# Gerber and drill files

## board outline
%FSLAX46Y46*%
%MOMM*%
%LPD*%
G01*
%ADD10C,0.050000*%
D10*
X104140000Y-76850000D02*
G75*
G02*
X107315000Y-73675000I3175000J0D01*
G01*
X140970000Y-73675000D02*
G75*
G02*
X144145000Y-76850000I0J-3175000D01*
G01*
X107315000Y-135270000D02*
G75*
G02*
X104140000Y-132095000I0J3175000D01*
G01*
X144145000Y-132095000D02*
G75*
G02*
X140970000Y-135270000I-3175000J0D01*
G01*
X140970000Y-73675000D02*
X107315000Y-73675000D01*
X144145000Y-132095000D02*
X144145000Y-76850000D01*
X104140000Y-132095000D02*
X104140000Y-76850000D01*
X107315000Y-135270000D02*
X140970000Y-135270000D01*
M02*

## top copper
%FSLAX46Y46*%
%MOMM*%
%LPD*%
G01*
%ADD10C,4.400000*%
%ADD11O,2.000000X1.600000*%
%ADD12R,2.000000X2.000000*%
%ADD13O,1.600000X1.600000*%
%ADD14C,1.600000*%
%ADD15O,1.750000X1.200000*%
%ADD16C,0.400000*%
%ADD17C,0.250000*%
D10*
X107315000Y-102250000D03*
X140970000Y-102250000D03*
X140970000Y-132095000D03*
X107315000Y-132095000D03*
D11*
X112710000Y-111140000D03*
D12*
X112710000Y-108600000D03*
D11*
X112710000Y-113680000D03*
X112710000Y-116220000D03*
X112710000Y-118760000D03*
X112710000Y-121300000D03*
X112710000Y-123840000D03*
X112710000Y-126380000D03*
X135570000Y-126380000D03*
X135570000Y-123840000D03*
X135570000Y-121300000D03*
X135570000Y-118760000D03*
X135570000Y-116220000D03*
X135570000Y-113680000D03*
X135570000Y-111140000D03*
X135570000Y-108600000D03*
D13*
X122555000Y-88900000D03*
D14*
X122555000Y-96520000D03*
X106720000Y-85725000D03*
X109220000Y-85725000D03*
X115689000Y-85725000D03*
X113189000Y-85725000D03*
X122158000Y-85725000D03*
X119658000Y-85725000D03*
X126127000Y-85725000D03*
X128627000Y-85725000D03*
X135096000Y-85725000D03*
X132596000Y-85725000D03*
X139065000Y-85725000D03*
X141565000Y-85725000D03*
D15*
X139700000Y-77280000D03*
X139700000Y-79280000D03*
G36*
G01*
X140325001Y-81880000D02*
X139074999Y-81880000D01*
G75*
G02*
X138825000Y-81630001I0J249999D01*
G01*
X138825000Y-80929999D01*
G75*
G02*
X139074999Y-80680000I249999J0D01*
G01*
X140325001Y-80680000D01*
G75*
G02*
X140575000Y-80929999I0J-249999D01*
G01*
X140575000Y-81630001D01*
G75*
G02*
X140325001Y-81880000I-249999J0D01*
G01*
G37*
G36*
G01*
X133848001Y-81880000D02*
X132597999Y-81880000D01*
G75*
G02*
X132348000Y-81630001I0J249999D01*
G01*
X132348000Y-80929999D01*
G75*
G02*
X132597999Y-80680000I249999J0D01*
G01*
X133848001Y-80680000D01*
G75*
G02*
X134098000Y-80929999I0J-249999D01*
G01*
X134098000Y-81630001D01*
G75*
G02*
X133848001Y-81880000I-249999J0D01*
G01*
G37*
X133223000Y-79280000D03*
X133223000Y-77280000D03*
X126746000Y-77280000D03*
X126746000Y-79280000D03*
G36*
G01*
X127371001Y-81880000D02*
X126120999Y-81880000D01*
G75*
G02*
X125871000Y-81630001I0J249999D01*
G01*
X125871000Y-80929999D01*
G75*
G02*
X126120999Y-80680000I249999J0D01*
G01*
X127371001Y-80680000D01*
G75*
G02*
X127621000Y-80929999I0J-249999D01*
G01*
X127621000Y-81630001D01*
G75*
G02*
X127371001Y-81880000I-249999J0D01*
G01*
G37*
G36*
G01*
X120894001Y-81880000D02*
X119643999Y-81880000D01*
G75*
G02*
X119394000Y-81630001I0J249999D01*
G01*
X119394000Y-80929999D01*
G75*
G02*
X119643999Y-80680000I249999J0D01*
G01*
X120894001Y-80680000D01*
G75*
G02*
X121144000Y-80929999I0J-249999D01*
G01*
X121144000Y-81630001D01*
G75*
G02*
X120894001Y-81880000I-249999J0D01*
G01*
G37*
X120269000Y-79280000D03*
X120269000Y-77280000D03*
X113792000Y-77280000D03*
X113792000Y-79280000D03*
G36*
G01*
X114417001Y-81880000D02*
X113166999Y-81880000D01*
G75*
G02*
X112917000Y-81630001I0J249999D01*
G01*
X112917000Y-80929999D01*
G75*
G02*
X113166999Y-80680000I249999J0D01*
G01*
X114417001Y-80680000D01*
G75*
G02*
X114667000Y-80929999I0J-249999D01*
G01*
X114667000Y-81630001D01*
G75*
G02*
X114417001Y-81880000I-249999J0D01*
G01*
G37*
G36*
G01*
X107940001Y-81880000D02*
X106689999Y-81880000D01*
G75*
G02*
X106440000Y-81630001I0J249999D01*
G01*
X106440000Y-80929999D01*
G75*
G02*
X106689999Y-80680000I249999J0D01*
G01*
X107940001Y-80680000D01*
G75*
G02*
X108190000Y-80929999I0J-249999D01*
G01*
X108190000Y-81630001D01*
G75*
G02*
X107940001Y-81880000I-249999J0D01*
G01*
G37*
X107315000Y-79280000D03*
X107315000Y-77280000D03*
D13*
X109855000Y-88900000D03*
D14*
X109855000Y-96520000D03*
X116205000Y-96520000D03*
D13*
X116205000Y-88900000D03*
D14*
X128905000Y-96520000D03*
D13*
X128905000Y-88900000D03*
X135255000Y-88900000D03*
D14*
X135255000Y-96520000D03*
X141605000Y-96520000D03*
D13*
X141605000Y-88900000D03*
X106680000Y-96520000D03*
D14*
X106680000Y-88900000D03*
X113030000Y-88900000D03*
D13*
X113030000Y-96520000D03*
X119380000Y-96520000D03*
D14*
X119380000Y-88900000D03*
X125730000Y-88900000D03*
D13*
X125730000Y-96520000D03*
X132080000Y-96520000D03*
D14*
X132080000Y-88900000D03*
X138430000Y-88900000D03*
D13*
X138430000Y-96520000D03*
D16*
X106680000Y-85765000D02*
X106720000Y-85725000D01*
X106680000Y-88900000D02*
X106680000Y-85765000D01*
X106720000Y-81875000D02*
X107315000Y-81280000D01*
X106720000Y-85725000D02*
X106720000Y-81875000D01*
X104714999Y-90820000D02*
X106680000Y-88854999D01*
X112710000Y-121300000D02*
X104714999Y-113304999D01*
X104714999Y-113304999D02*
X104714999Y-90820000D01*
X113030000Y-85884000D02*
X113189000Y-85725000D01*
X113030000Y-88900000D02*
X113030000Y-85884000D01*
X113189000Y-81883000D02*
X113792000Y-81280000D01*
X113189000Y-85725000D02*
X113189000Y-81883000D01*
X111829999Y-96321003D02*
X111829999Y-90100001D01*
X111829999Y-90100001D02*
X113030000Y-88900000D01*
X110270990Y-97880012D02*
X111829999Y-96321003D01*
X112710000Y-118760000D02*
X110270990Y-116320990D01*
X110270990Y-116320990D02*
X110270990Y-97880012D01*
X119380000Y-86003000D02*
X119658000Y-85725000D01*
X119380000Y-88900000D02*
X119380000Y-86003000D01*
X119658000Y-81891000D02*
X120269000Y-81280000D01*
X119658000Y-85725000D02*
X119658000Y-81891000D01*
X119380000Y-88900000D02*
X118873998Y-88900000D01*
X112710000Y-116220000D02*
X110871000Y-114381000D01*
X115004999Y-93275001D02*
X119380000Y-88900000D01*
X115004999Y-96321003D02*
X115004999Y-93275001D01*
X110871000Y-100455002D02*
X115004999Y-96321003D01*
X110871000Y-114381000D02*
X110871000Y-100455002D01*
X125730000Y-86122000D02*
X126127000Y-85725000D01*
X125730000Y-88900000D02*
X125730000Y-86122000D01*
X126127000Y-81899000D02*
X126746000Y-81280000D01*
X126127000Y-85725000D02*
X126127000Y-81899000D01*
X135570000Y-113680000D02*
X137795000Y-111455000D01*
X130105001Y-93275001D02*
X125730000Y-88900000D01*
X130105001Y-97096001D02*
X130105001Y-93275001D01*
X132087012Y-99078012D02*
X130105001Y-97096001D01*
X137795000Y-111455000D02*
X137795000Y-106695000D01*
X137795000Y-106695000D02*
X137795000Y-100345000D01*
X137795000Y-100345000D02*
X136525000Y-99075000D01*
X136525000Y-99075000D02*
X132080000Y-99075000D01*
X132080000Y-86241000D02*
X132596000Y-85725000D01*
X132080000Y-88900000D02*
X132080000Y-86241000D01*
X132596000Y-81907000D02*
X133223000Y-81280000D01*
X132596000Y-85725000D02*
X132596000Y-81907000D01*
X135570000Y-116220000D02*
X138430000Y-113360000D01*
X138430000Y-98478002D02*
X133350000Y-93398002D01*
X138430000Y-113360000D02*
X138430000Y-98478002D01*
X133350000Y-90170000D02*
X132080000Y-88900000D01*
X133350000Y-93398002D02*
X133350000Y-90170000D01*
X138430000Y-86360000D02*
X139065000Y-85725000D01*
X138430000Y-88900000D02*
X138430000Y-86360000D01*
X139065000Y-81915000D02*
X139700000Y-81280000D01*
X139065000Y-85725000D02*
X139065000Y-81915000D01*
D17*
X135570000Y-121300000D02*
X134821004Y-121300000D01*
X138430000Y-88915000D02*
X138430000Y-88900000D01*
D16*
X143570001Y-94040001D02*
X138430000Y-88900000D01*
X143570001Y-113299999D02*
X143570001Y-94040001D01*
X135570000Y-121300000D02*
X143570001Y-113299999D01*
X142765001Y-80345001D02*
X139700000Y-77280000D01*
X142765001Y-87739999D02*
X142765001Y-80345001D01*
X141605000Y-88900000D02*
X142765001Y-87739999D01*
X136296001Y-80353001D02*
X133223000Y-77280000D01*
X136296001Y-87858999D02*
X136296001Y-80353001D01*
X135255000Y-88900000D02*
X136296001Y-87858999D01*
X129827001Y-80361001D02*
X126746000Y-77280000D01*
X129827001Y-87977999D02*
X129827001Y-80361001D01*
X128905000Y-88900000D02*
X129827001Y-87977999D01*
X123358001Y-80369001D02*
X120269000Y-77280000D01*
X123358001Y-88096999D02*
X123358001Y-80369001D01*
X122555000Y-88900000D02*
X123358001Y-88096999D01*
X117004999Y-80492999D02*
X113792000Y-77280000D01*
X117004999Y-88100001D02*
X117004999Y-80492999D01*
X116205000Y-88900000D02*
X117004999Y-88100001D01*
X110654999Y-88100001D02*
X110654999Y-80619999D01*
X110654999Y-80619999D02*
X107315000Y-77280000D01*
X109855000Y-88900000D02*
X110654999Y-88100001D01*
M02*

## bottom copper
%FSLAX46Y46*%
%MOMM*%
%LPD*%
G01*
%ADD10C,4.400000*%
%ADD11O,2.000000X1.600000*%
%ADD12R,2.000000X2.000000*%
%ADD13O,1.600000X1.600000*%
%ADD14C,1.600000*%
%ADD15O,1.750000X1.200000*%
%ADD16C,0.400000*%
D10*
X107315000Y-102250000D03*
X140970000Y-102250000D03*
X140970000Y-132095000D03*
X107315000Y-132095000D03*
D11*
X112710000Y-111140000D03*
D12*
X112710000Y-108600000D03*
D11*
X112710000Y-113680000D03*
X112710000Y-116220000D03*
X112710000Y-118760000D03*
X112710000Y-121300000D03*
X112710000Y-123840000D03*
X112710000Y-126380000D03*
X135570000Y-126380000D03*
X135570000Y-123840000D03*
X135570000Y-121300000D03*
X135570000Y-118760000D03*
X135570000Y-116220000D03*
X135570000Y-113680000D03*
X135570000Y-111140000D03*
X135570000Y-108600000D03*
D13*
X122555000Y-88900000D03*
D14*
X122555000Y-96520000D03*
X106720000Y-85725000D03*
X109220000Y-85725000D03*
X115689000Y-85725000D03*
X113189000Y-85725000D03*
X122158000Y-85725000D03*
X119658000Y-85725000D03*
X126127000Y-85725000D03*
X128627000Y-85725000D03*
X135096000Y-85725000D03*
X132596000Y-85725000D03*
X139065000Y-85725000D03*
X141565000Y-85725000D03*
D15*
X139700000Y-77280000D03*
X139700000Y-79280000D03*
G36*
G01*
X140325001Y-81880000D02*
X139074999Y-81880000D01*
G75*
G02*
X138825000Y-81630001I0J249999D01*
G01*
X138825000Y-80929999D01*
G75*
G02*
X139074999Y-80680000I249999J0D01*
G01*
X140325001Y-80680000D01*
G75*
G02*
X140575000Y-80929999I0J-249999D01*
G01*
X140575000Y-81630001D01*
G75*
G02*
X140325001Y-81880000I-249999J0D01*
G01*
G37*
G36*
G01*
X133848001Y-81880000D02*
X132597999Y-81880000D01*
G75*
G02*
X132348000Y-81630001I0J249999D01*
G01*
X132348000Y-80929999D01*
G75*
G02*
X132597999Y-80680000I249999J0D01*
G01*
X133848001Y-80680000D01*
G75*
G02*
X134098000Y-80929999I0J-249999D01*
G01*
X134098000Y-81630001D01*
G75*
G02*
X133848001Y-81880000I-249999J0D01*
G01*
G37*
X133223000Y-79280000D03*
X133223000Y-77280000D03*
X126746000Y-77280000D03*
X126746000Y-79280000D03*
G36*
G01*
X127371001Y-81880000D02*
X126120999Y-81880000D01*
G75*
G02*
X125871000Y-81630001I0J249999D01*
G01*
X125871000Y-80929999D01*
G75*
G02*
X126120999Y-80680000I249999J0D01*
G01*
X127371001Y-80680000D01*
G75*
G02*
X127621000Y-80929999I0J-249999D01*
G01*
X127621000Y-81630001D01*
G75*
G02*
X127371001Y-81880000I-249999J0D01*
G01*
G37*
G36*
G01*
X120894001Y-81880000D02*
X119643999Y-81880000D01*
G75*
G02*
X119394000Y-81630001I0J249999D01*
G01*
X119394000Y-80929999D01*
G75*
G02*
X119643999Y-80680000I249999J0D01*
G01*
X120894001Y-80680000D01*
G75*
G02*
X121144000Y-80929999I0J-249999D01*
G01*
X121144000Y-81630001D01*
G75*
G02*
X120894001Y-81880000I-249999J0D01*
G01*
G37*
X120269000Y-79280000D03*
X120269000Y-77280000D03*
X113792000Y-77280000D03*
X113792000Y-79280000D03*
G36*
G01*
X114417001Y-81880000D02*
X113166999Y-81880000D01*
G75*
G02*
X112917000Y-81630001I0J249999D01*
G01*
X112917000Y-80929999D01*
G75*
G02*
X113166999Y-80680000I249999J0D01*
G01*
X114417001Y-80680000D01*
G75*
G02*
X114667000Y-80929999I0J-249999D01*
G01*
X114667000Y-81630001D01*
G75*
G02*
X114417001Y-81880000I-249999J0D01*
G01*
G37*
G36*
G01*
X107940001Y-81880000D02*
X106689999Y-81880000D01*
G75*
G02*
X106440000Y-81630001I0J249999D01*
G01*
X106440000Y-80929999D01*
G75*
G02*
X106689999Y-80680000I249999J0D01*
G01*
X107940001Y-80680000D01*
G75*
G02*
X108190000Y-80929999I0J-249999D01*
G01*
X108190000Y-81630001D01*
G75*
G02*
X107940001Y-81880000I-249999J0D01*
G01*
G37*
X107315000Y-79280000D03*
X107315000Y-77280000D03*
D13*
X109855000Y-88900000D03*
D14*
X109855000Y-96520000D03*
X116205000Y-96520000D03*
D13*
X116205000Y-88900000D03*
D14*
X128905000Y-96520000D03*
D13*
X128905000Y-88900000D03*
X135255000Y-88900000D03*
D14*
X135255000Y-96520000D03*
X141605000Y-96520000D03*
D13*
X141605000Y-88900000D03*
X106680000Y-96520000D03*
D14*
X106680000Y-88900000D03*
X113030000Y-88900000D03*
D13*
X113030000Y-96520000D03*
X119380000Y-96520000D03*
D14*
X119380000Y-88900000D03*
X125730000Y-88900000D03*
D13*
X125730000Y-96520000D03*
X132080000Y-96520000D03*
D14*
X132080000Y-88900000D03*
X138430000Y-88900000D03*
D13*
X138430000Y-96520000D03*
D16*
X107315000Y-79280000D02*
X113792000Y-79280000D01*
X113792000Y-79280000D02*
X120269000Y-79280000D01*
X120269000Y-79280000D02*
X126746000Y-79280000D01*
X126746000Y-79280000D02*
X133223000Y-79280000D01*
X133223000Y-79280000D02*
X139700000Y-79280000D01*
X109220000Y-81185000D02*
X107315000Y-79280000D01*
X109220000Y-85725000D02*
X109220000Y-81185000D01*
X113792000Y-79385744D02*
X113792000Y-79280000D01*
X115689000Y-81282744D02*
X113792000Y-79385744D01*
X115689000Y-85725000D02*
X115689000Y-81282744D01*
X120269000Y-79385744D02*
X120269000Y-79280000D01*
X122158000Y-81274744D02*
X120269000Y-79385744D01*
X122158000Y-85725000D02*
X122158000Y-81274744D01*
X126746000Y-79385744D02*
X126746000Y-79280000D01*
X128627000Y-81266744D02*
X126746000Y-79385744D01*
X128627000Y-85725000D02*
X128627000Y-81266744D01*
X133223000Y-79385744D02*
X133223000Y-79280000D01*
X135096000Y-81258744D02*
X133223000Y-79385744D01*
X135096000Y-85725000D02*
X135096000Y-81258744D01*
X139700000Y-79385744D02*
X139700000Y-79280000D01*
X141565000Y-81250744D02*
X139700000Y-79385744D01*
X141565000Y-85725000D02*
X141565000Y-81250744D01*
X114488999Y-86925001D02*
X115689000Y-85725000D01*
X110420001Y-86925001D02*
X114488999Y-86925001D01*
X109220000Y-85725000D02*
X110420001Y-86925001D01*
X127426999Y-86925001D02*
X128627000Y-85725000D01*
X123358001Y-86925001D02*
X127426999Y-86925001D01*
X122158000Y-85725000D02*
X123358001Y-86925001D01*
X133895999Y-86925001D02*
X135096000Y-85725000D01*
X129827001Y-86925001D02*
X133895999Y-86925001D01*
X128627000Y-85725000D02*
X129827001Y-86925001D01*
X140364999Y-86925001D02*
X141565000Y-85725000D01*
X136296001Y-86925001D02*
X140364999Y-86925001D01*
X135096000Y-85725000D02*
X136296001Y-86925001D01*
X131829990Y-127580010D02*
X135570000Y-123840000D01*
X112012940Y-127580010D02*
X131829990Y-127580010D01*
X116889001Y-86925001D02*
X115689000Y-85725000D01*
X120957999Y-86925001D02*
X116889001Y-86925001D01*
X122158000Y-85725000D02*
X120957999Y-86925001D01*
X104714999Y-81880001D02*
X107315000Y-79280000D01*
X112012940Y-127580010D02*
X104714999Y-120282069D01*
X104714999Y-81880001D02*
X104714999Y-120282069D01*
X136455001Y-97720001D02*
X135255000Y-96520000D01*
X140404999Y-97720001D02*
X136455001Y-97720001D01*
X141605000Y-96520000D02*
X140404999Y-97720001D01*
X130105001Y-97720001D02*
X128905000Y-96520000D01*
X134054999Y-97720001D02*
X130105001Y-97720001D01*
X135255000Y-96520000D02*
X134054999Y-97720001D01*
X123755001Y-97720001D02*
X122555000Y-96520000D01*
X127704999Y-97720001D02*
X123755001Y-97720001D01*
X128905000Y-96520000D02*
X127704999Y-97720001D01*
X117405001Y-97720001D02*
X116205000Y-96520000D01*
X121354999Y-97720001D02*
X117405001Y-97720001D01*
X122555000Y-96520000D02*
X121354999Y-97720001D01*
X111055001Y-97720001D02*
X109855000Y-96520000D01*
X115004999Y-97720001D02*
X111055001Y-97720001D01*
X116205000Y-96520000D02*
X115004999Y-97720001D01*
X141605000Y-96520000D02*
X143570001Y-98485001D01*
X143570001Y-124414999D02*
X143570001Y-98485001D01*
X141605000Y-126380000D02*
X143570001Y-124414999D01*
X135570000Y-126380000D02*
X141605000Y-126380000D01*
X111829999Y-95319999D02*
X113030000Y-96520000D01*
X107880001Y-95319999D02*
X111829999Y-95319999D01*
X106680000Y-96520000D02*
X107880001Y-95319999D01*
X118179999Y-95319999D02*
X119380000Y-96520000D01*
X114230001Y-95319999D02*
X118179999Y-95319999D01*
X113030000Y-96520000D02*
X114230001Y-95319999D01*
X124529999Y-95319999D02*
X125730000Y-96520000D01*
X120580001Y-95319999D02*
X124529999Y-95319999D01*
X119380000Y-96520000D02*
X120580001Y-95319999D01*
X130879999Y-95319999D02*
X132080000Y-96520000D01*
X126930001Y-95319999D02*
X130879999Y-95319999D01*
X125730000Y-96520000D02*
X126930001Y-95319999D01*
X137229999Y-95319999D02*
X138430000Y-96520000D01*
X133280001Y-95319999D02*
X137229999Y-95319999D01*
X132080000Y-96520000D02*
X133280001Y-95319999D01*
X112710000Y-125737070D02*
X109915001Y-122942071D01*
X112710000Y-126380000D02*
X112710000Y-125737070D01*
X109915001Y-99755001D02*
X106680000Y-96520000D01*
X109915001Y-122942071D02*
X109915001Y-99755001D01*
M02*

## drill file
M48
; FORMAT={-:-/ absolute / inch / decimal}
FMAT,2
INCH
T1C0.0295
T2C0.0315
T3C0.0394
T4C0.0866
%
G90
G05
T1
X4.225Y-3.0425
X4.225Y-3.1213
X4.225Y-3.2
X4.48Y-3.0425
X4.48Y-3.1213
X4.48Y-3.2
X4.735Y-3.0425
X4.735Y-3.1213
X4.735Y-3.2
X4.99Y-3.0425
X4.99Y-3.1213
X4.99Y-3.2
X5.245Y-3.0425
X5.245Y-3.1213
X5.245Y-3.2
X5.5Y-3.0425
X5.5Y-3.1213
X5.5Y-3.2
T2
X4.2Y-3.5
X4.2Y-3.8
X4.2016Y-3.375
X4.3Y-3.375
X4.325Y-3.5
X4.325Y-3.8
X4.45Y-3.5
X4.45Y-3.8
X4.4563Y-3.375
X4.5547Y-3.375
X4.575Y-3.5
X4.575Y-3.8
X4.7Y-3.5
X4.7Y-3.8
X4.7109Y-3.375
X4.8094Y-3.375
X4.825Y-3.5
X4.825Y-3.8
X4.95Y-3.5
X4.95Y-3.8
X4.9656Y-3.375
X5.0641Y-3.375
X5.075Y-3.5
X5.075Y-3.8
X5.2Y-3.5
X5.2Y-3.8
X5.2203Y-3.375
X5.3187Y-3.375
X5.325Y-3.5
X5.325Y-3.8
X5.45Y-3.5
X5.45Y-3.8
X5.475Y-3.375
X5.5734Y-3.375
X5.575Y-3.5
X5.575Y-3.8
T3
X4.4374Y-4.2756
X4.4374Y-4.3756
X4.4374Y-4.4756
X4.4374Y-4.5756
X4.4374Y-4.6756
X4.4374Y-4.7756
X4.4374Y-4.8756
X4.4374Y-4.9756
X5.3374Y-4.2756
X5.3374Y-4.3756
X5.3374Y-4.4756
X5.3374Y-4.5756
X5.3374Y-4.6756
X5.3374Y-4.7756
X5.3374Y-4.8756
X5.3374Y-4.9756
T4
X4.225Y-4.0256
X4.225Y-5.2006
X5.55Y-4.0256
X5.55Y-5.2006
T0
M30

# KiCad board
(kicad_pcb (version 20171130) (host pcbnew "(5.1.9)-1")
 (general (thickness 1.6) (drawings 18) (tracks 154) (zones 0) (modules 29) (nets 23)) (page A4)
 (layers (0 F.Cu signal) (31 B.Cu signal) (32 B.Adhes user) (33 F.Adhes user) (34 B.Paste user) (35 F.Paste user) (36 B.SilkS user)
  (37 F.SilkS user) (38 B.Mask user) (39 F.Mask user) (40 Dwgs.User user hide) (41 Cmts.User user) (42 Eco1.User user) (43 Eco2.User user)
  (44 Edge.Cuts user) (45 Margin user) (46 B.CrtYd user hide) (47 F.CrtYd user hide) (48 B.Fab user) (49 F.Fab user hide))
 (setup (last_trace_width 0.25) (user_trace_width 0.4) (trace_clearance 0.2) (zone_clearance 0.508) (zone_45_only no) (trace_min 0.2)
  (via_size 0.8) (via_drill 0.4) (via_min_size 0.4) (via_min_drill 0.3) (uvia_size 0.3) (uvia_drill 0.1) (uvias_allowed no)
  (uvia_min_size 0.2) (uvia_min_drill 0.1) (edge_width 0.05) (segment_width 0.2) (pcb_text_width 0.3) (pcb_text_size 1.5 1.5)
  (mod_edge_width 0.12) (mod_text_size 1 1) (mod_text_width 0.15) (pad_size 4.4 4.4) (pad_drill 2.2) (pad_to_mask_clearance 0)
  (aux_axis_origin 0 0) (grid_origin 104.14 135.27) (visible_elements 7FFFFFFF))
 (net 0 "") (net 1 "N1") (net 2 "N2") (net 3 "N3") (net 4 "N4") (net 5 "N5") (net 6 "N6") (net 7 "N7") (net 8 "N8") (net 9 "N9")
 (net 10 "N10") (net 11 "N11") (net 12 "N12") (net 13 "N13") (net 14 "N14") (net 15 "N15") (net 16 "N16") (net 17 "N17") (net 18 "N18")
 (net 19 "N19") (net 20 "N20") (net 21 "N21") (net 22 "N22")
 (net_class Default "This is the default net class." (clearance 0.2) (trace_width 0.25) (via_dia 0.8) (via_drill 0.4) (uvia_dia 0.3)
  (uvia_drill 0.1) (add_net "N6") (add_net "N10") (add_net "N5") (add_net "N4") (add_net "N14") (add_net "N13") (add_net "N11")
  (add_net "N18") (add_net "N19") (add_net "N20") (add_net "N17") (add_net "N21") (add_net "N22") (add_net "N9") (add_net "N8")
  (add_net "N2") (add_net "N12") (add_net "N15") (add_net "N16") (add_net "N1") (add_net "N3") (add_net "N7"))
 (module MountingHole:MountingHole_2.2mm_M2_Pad (layer F.Cu) (at 107.315 102.25)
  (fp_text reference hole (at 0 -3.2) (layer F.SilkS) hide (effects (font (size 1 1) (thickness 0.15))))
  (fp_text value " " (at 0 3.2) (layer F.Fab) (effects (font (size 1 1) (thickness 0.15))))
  (pad 4 thru_hole circle (at 0 0) (size 4.4 4.4) (drill 2.2) (layers *.Cu *.Mask)))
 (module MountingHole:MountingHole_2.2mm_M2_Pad (layer F.Cu) (at 140.97 102.25)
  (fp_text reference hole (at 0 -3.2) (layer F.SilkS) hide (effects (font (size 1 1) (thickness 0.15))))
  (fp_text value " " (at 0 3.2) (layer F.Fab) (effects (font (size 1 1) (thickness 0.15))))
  (pad 3 thru_hole circle (at 0 0) (size 4.4 4.4) (drill 2.2) (layers *.Cu *.Mask)))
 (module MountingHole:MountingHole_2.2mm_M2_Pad (layer F.Cu) (at 140.97 132.095)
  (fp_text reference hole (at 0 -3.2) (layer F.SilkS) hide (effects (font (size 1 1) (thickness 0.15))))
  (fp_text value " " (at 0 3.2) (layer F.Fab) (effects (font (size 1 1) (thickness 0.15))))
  (pad 2 thru_hole circle (at 0 0) (size 4.4 4.4) (drill 2.2) (layers *.Cu *.Mask)))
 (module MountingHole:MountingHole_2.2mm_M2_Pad (layer F.Cu) (at 107.315 132.095)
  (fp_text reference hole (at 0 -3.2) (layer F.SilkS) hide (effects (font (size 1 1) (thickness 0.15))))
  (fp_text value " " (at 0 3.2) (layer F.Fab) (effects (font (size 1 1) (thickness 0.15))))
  (pad 1 thru_hole circle (at 0 0) (size 4.4 4.4) (drill 2.2) (layers *.Cu *.Mask)))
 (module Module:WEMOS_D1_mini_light (layer F.Cu) (at 112.71 108.6)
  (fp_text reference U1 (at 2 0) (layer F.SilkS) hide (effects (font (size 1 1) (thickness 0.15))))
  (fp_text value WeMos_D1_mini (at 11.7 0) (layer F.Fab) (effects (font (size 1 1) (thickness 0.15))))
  (pad 2 thru_hole oval (at 0 2.54) (size 2 1.6) (drill 1) (layers *.Cu *.Mask) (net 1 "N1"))
  (pad 1 thru_hole rect (at 0 0) (size 2 2) (drill 1) (layers *.Cu *.Mask) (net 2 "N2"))
  (pad 3 thru_hole oval (at 0 5.08) (size 2 1.6) (drill 1) (layers *.Cu *.Mask) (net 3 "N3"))
  (pad 4 thru_hole oval (at 0 7.62) (size 2 1.6) (drill 1) (layers *.Cu *.Mask) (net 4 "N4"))
  (pad 5 thru_hole oval (at 0 10.16) (size 2 1.6) (drill 1) (layers *.Cu *.Mask) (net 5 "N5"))
  (pad 6 thru_hole oval (at 0 12.7) (size 2 1.6) (drill 1) (layers *.Cu *.Mask) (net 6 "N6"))
  (pad 7 thru_hole oval (at 0 15.24) (size 2 1.6) (drill 1) (layers *.Cu *.Mask) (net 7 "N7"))
  (pad 8 thru_hole oval (at 0 17.78) (size 2 1.6) (drill 1) (layers *.Cu *.Mask) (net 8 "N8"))
  (pad 9 thru_hole oval (at 22.86 17.78) (size 2 1.6) (drill 1) (layers *.Cu *.Mask) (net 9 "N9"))
  (pad 10 thru_hole oval (at 22.86 15.24) (size 2 1.6) (drill 1) (layers *.Cu *.Mask) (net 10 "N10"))
  (pad 11 thru_hole oval (at 22.86 12.7) (size 2 1.6) (drill 1) (layers *.Cu *.Mask) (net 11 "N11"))
  (pad 12 thru_hole oval (at 22.86 10.16) (size 2 1.6) (drill 1) (layers *.Cu *.Mask) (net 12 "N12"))
  (pad 13 thru_hole oval (at 22.86 7.62) (size 2 1.6) (drill 1) (layers *.Cu *.Mask) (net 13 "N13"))
  (pad 14 thru_hole oval (at 22.86 5.08) (size 2 1.6) (drill 1) (layers *.Cu *.Mask) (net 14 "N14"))
  (pad 15 thru_hole oval (at 22.86 2.54) (size 2 1.6) (drill 1) (layers *.Cu *.Mask) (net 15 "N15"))
  (pad 16 thru_hole oval (at 22.86 0) (size 2 1.6) (drill 1) (layers *.Cu *.Mask) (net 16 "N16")))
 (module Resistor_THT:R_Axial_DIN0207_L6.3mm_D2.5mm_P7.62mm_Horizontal (layer F.Cu) (at 122.555 96.52 90)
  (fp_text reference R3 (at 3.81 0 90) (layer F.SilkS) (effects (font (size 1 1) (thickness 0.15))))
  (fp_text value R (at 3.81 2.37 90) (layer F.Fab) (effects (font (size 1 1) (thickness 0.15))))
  (pad 2 thru_hole oval (at 7.62 0 90) (size 1.6 1.6) (drill 0.8) (layers *.Cu *.Mask) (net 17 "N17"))
  (pad 1 thru_hole circle (at 0 0 90) (size 1.6 1.6) (drill 0.8) (layers *.Cu *.Mask) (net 9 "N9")))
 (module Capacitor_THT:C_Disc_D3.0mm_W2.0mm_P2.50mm (layer F.Cu) (at 106.72 85.725)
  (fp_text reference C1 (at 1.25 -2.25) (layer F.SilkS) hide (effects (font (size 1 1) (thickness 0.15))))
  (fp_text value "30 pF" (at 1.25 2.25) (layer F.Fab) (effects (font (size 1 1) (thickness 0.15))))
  (pad 1 thru_hole circle (at 0 0) (size 1.6 1.6) (drill 0.8) (layers *.Cu *.Mask) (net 6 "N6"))
  (pad 2 thru_hole circle (at 2.5 0) (size 1.6 1.6) (drill 0.8) (layers *.Cu *.Mask) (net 10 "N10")))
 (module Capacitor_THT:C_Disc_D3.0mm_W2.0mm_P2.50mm (layer F.Cu) (at 113.189 85.725)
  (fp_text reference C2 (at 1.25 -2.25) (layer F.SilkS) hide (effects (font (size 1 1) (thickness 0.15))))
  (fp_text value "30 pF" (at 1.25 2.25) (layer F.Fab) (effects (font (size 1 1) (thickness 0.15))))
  (pad 2 thru_hole circle (at 2.5 0) (size 1.6 1.6) (drill 0.8) (layers *.Cu *.Mask) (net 10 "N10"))
  (pad 1 thru_hole circle (at 0 0) (size 1.6 1.6) (drill 0.8) (layers *.Cu *.Mask) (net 5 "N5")))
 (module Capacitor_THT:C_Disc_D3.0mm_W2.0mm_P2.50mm (layer F.Cu) (at 119.658 85.725)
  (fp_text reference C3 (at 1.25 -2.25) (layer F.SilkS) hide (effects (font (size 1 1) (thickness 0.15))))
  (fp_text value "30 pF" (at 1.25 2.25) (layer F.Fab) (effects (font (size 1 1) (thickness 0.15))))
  (pad 2 thru_hole circle (at 2.5 0) (size 1.6 1.6) (drill 0.8) (layers *.Cu *.Mask) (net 10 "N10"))
  (pad 1 thru_hole circle (at 0 0) (size 1.6 1.6) (drill 0.8) (layers *.Cu *.Mask) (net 4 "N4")))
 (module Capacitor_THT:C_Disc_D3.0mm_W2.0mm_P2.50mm (layer F.Cu) (at 126.127 85.725)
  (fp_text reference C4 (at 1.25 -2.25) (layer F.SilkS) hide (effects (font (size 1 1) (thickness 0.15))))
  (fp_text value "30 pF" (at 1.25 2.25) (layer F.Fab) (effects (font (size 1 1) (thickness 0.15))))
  (pad 1 thru_hole circle (at 0 0) (size 1.6 1.6) (drill 0.8) (layers *.Cu *.Mask) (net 14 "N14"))
  (pad 2 thru_hole circle (at 2.5 0) (size 1.6 1.6) (drill 0.8) (layers *.Cu *.Mask) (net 10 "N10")))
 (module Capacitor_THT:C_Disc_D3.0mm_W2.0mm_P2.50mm (layer F.Cu) (at 132.596 85.725)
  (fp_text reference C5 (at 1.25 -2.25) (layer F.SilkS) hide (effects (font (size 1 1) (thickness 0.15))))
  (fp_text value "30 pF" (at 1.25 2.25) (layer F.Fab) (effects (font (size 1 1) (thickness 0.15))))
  (pad 2 thru_hole circle (at 2.5 0) (size 1.6 1.6) (drill 0.8) (layers *.Cu *.Mask) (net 10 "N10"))
  (pad 1 thru_hole circle (at 0 0) (size 1.6 1.6) (drill 0.8) (layers *.Cu *.Mask) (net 13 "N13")))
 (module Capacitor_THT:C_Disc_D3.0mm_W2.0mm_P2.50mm (layer F.Cu) (at 139.065 85.725)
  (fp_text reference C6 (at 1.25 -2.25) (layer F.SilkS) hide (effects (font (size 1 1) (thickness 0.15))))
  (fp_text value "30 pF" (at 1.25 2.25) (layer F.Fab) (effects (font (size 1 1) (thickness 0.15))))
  (pad 1 thru_hole circle (at 0 0) (size 1.6 1.6) (drill 0.8) (layers *.Cu *.Mask) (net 11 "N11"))
  (pad 2 thru_hole circle (at 2.5 0) (size 1.6 1.6) (drill 0.8) (layers *.Cu *.Mask) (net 10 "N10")))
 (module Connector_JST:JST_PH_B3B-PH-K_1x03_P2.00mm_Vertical (layer F.Cu) (at 139.7 81.28 90)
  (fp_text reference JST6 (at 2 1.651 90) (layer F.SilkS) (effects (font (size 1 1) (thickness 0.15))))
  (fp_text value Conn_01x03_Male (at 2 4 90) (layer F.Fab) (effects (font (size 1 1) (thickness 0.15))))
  (pad 3 thru_hole oval (at 4 0 90) (size 1.2 1.75) (drill 0.75) (layers *.Cu *.Mask) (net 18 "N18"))
  (pad 2 thru_hole oval (at 2 0 90) (size 1.2 1.75) (drill 0.75) (layers *.Cu *.Mask) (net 10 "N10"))
  (pad 1 thru_hole roundrect (at 0 0 90) (size 1.2 1.75) (drill 0.75) (layers *.Cu *.Mask) (roundrect_rratio 0.2083325) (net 11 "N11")))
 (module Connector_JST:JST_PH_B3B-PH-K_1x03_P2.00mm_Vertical (layer F.Cu) (at 133.223 81.28 90)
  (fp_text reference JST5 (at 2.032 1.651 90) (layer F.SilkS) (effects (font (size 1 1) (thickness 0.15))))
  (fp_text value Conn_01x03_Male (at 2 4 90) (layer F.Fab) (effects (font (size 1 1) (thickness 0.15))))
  (pad 1 thru_hole roundrect (at 0 0 90) (size 1.2 1.75) (drill 0.75) (layers *.Cu *.Mask) (roundrect_rratio 0.2083325) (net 13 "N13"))
  (pad 2 thru_hole oval (at 2 0 90) (size 1.2 1.75) (drill 0.75) (layers *.Cu *.Mask) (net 10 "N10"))
  (pad 3 thru_hole oval (at 4 0 90) (size 1.2 1.75) (drill 0.75) (layers *.Cu *.Mask) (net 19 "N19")))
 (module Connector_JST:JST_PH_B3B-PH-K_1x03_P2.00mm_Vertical (layer F.Cu) (at 126.746 81.28 90)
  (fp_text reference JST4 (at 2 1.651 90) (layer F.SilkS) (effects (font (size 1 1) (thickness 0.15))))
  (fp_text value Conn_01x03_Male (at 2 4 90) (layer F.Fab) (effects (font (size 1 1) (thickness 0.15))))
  (pad 3 thru_hole oval (at 4 0 90) (size 1.2 1.75) (drill 0.75) (layers *.Cu *.Mask) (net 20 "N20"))
  (pad 2 thru_hole oval (at 2 0 90) (size 1.2 1.75) (drill 0.75) (layers *.Cu *.Mask) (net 10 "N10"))
  (pad 1 thru_hole roundrect (at 0 0 90) (size 1.2 1.75) (drill 0.75) (layers *.Cu *.Mask) (roundrect_rratio 0.2083325) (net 14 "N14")))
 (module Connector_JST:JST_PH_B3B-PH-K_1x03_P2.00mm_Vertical (layer F.Cu) (at 120.269 81.28 90)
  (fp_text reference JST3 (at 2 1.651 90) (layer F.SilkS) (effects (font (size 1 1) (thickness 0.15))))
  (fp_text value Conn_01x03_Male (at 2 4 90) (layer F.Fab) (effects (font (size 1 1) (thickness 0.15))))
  (pad 1 thru_hole roundrect (at 0 0 90) (size 1.2 1.75) (drill 0.75) (layers *.Cu *.Mask) (roundrect_rratio 0.2083325) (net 4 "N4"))
  (pad 2 thru_hole oval (at 2 0 90) (size 1.2 1.75) (drill 0.75) (layers *.Cu *.Mask) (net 10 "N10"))
  (pad 3 thru_hole oval (at 4 0 90) (size 1.2 1.75) (drill 0.75) (layers *.Cu *.Mask) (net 17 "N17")))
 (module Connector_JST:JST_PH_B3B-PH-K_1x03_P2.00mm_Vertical (layer F.Cu) (at 113.792 81.28 90)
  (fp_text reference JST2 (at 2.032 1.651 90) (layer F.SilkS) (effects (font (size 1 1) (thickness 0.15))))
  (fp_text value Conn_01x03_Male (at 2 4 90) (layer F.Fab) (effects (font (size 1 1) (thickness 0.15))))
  (pad 3 thru_hole oval (at 4 0 90) (size 1.2 1.75) (drill 0.75) (layers *.Cu *.Mask) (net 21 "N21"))
  (pad 2 thru_hole oval (at 2 0 90) (size 1.2 1.75) (drill 0.75) (layers *.Cu *.Mask) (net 10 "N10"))
  (pad 1 thru_hole roundrect (at 0 0 90) (size 1.2 1.75) (drill 0.75) (layers *.Cu *.Mask) (roundrect_rratio 0.2083325) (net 5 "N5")))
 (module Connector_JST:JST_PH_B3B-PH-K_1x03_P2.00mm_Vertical (layer F.Cu) (at 107.315 81.28 90)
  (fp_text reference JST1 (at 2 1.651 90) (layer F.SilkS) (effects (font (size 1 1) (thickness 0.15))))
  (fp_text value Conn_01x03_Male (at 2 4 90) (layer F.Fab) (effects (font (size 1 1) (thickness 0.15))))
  (pad 3 thru_hole oval (at 4 0 90) (size 1.2 1.75) (drill 0.75) (layers *.Cu *.Mask) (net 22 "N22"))
  (pad 2 thru_hole oval (at 2 0 90) (size 1.2 1.75) (drill 0.75) (layers *.Cu *.Mask) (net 10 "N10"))
  (pad 1 thru_hole roundrect (at 0 0 90) (size 1.2 1.75) (drill 0.75) (layers *.Cu *.Mask) (roundrect_rratio 0.2083325) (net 6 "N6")))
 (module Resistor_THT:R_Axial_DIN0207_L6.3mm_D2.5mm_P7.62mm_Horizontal (layer F.Cu) (at 109.855 96.52 90)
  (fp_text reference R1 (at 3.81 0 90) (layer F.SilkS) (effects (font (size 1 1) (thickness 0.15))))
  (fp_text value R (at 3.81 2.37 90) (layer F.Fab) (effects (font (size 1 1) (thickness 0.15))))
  (pad 2 thru_hole oval (at 7.62 0 90) (size 1.6 1.6) (drill 0.8) (layers *.Cu *.Mask) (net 22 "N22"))
  (pad 1 thru_hole circle (at 0 0 90) (size 1.6 1.6) (drill 0.8) (layers *.Cu *.Mask) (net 9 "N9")))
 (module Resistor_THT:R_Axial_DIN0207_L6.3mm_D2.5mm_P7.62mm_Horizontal (layer F.Cu) (at 116.205 96.52 90)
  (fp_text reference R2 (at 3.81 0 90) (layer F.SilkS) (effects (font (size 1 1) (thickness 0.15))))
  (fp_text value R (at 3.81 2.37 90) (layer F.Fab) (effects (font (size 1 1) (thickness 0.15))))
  (pad 1 thru_hole circle (at 0 0 90) (size 1.6 1.6) (drill 0.8) (layers *.Cu *.Mask) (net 9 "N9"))
  (pad 2 thru_hole oval (at 7.62 0 90) (size 1.6 1.6) (drill 0.8) (layers *.Cu *.Mask) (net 21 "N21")))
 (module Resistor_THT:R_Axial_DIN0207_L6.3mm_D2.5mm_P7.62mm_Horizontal (layer F.Cu) (at 128.905 96.52 90)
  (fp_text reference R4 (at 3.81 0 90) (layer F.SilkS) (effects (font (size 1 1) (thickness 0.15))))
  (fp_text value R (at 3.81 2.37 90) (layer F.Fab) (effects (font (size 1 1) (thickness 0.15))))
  (pad 1 thru_hole circle (at 0 0 90) (size 1.6 1.6) (drill 0.8) (layers *.Cu *.Mask) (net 9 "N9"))
  (pad 2 thru_hole oval (at 7.62 0 90) (size 1.6 1.6) (drill 0.8) (layers *.Cu *.Mask) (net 20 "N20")))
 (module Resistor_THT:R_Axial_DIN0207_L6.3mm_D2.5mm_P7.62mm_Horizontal (layer F.Cu) (at 135.255 96.52 90)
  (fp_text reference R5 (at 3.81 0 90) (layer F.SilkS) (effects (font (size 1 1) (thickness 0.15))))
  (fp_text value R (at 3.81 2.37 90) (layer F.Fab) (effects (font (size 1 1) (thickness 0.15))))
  (pad 2 thru_hole oval (at 7.62 0 90) (size 1.6 1.6) (drill 0.8) (layers *.Cu *.Mask) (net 19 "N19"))
  (pad 1 thru_hole circle (at 0 0 90) (size 1.6 1.6) (drill 0.8) (layers *.Cu *.Mask) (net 9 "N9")))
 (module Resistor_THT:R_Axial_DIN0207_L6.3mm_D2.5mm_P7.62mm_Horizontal (layer F.Cu) (at 141.605 96.52 90)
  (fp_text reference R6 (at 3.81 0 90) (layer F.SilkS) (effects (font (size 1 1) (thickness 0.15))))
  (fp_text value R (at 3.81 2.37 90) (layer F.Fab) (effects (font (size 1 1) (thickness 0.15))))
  (pad 1 thru_hole circle (at 0 0 90) (size 1.6 1.6) (drill 0.8) (layers *.Cu *.Mask) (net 9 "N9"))
  (pad 2 thru_hole oval (at 7.62 0 90) (size 1.6 1.6) (drill 0.8) (layers *.Cu *.Mask) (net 18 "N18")))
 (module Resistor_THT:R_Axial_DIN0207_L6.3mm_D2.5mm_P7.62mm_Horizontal (layer F.Cu) (at 106.68 88.9 270)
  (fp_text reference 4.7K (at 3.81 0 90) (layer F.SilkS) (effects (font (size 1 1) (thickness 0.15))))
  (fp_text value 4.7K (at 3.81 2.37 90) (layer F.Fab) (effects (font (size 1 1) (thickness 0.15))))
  (pad 2 thru_hole oval (at 7.62 0 270) (size 1.6 1.6) (drill 0.8) (layers *.Cu *.Mask) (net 8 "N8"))
  (pad 1 thru_hole circle (at 0 0 270) (size 1.6 1.6) (drill 0.8) (layers *.Cu *.Mask) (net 6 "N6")))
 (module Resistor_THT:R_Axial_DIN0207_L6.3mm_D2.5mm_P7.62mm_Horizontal (layer F.Cu) (at 113.03 88.9 270)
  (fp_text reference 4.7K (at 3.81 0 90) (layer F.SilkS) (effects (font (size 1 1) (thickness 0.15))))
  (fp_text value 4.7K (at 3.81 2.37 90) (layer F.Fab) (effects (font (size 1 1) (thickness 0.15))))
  (pad 1 thru_hole circle (at 0 0 270) (size 1.6 1.6) (drill 0.8) (layers *.Cu *.Mask) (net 5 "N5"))
  (pad 2 thru_hole oval (at 7.62 0 270) (size 1.6 1.6) (drill 0.8) (layers *.Cu *.Mask) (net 8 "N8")))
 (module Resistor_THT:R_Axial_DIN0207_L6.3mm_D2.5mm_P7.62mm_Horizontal (layer F.Cu) (at 119.38 88.9 270)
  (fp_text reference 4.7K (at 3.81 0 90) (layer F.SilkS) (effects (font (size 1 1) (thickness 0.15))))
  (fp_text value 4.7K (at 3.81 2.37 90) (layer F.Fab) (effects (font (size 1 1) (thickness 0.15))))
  (pad 2 thru_hole oval (at 7.62 0 270) (size 1.6 1.6) (drill 0.8) (layers *.Cu *.Mask) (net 8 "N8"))
  (pad 1 thru_hole circle (at 0 0 270) (size 1.6 1.6) (drill 0.8) (layers *.Cu *.Mask) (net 4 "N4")))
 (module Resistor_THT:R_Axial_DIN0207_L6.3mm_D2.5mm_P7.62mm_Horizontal (layer F.Cu) (at 125.73 88.9 270)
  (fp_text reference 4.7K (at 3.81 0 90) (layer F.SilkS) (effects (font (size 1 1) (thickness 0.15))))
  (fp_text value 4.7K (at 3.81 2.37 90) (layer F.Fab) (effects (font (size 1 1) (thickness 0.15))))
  (pad 1 thru_hole circle (at 0 0 270) (size 1.6 1.6) (drill 0.8) (layers *.Cu *.Mask) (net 14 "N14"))
  (pad 2 thru_hole oval (at 7.62 0 270) (size 1.6 1.6) (drill 0.8) (layers *.Cu *.Mask) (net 8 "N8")))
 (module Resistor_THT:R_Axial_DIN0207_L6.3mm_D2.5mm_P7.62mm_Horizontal (layer F.Cu) (at 132.08 88.9 270)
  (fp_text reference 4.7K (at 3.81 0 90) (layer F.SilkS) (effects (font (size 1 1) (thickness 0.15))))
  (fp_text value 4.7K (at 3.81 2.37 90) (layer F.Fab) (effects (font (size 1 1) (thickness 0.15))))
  (pad 2 thru_hole oval (at 7.62 0 270) (size 1.6 1.6) (drill 0.8) (layers *.Cu *.Mask) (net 8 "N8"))
  (pad 1 thru_hole circle (at 0 0 270) (size 1.6 1.6) (drill 0.8) (layers *.Cu *.Mask) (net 13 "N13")))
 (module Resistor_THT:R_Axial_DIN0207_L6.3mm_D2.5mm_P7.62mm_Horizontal (layer F.Cu) (at 138.43 88.9 270)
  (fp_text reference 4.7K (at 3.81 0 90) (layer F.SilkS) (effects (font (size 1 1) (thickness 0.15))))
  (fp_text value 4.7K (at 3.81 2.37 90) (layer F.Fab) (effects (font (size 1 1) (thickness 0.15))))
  (pad 1 thru_hole circle (at 0 0 270) (size 1.6 1.6) (drill 0.8) (layers *.Cu *.Mask) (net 11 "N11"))
  (pad 2 thru_hole oval (at 7.62 0 270) (size 1.6 1.6) (drill 0.8) (layers *.Cu *.Mask) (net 8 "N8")))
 (gr_arc (start 107.315 76.85) (end 107.315 73.675) (angle -90) (layer Edge.Cuts) (width 0.05))
 (gr_arc (start 140.97 76.85) (end 144.145 76.85) (angle -90) (layer Edge.Cuts) (width 0.05))
 (gr_arc (start 107.315 132.095) (end 104.14 132.095) (angle -90) (layer Edge.Cuts) (width 0.05))
 (gr_arc (start 140.97 132.095) (end 140.97 135.27) (angle -90) (layer Edge.Cuts) (width 0.05))
 (gr_line (start 140.97 73.675) (end 107.315 73.675) (layer Edge.Cuts) (width 0.05))
 (gr_line (start 144.145 132.095) (end 144.145 76.85) (layer Edge.Cuts) (width 0.05))
 (gr_line (start 104.14 132.095) (end 104.14 76.85) (layer Edge.Cuts) (width 0.05))
 (gr_line (start 107.315 135.27) (end 140.97 135.27) (layer Edge.Cuts) (width 0.05))
 (segment (start 106.68 85.765) (end 106.72 85.725) (width 0.4) (layer F.Cu) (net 6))
 (segment (start 106.68 88.9) (end 106.68 85.765) (width 0.4) (layer F.Cu) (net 6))
 (segment (start 106.72 81.875) (end 107.315 81.28) (width 0.4) (layer F.Cu) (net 6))
 (segment (start 106.72 85.725) (end 106.72 81.875) (width 0.4) (layer F.Cu) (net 6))
 (segment (start 104.714999 90.82) (end 106.68 88.854999) (width 0.4) (layer F.Cu) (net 6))
 (segment (start 112.71 121.3) (end 104.714999 113.304999) (width 0.4) (layer F.Cu) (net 6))
 (segment (start 104.714999 113.304999) (end 104.714999 90.82) (width 0.4) (layer F.Cu) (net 6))
 (segment (start 107.315 79.28) (end 113.792 79.28) (width 0.4) (layer B.Cu) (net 10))
 (segment (start 113.792 79.28) (end 120.269 79.28) (width 0.4) (layer B.Cu) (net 10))
 (segment (start 120.269 79.28) (end 126.746 79.28) (width 0.4) (layer B.Cu) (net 10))
 (segment (start 126.746 79.28) (end 133.223 79.28) (width 0.4) (layer B.Cu) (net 10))
 (segment (start 133.223 79.28) (end 139.7 79.28) (width 0.4) (layer B.Cu) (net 10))
 (segment (start 109.22 81.185) (end 107.315 79.28) (width 0.4) (layer B.Cu) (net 10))
 (segment (start 109.22 85.725) (end 109.22 81.185) (width 0.4) (layer B.Cu) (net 10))
 (segment (start 113.792 79.385744) (end 113.792 79.28) (width 0.4) (layer B.Cu) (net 10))
 (segment (start 115.689 81.282744) (end 113.792 79.385744) (width 0.4) (layer B.Cu) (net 10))
 (segment (start 115.689 85.725) (end 115.689 81.282744) (width 0.4) (layer B.Cu) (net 10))
 (segment (start 120.269 79.385744) (end 120.269 79.28) (width 0.4) (layer B.Cu) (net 10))
 (segment (start 122.158 81.274744) (end 120.269 79.385744) (width 0.4) (layer B.Cu) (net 10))
 (segment (start 122.158 85.725) (end 122.158 81.274744) (width 0.4) (layer B.Cu) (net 10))
 (segment (start 126.746 79.385744) (end 126.746 79.28) (width 0.4) (layer B.Cu) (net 10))
 (segment (start 128.627 81.266744) (end 126.746 79.385744) (width 0.4) (layer B.Cu) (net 10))
 (segment (start 128.627 85.725) (end 128.627 81.266744) (width 0.4) (layer B.Cu) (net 10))
 (segment (start 133.223 79.385744) (end 133.223 79.28) (width 0.4) (layer B.Cu) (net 10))
 (segment (start 135.096 81.258744) (end 133.223 79.385744) (width 0.4) (layer B.Cu) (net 10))
 (segment (start 135.096 85.725) (end 135.096 81.258744) (width 0.4) (layer B.Cu) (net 10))
 (segment (start 139.7 79.385744) (end 139.7 79.28) (width 0.4) (layer B.Cu) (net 10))
 (segment (start 141.565 81.250744) (end 139.7 79.385744) (width 0.4) (layer B.Cu) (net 10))
 (segment (start 141.565 85.725) (end 141.565 81.250744) (width 0.4) (layer B.Cu) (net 10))
 (segment (start 114.488999 86.925001) (end 115.689 85.725) (width 0.4) (layer B.Cu) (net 10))
 (segment (start 110.420001 86.925001) (end 114.488999 86.925001) (width 0.4) (layer B.Cu) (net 10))
 (segment (start 109.22 85.725) (end 110.420001 86.925001) (width 0.4) (layer B.Cu) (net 10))
 (segment (start 127.426999 86.925001) (end 128.627 85.725) (width 0.4) (layer B.Cu) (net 10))
 (segment (start 123.358001 86.925001) (end 127.426999 86.925001) (width 0.4) (layer B.Cu) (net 10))
 (segment (start 122.158 85.725) (end 123.358001 86.925001) (width 0.4) (layer B.Cu) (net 10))
 (segment (start 133.895999 86.925001) (end 135.096 85.725) (width 0.4) (layer B.Cu) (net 10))
 (segment (start 129.827001 86.925001) (end 133.895999 86.925001) (width 0.4) (layer B.Cu) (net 10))
 (segment (start 128.627 85.725) (end 129.827001 86.925001) (width 0.4) (layer B.Cu) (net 10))
 (segment (start 140.364999 86.925001) (end 141.565 85.725) (width 0.4) (layer B.Cu) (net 10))
 (segment (start 136.296001 86.925001) (end 140.364999 86.925001) (width 0.4) (layer B.Cu) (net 10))
 (segment (start 135.096 85.725) (end 136.296001 86.925001) (width 0.4) (layer B.Cu) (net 10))
 (segment (start 131.82999 127.58001) (end 135.57 123.84) (width 0.4) (layer B.Cu) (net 10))
 (segment (start 112.01294 127.58001) (end 131.82999 127.58001) (width 0.4) (layer B.Cu) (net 10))
 (segment (start 116.889001 86.925001) (end 115.689 85.725) (width 0.4) (layer B.Cu) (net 10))
 (segment (start 120.957999 86.925001) (end 116.889001 86.925001) (width 0.4) (layer B.Cu) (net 10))
 (segment (start 122.158 85.725) (end 120.957999 86.925001) (width 0.4) (layer B.Cu) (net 10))
 (segment (start 104.714999 81.880001) (end 107.315 79.28) (width 0.4) (layer B.Cu) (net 10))
 (segment (start 112.01294 127.58001) (end 104.714999 120.282069) (width 0.4) (layer B.Cu) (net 10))
 (segment (start 104.714999 81.880001) (end 104.714999 120.282069) (width 0.4) (layer B.Cu) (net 10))
 (segment (start 113.03 85.884) (end 113.189 85.725) (width 0.4) (layer F.Cu) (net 5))
 (segment (start 113.03 88.9) (end 113.03 85.884) (width 0.4) (layer F.Cu) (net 5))
 (segment (start 113.189 81.883) (end 113.792 81.28) (width 0.4) (layer F.Cu) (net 5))
 (segment (start 113.189 85.725) (end 113.189 81.883) (width 0.4) (layer F.Cu) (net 5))
 (segment (start 111.829999 96.321003) (end 111.829999 90.100001) (width 0.4) (layer F.Cu) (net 5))
 (segment (start 111.829999 90.100001) (end 113.03 88.9) (width 0.4) (layer F.Cu) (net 5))
 (segment (start 110.27099 97.880012) (end 111.829999 96.321003) (width 0.4) (layer F.Cu) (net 5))
 (segment (start 112.71 118.76) (end 110.27099 116.32099) (width 0.4) (layer F.Cu) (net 5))
 (segment (start 110.27099 116.32099) (end 110.27099 97.880012) (width 0.4) (layer F.Cu) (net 5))
 (segment (start 119.38 86.003) (end 119.658 85.725) (width 0.4) (layer F.Cu) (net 4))
 (segment (start 119.38 88.9) (end 119.38 86.003) (width 0.4) (layer F.Cu) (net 4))
 (segment (start 119.658 81.891) (end 120.269 81.28) (width 0.4) (layer F.Cu) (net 4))
 (segment (start 119.658 85.725) (end 119.658 81.891) (width 0.4) (layer F.Cu) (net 4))
 (segment (start 119.38 88.9) (end 118.873998 88.9) (width 0.4) (layer F.Cu) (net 4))
 (segment (start 112.71 116.22) (end 110.871 114.381) (width 0.4) (layer F.Cu) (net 4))
 (segment (start 115.004999 93.275001) (end 119.38 88.9) (width 0.4) (layer F.Cu) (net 4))
 (segment (start 115.004999 96.321003) (end 115.004999 93.275001) (width 0.4) (layer F.Cu) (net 4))
 (segment (start 110.871 100.455002) (end 115.004999 96.321003) (width 0.4) (layer F.Cu) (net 4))
 (segment (start 110.871 114.381) (end 110.871 100.455002) (width 0.4) (layer F.Cu) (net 4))
 (segment (start 125.73 86.122) (end 126.127 85.725) (width 0.4) (layer F.Cu) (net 14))
 (segment (start 125.73 88.9) (end 125.73 86.122) (width 0.4) (layer F.Cu) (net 14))
 (segment (start 126.127 81.899) (end 126.746 81.28) (width 0.4) (layer F.Cu) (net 14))
 (segment (start 126.127 85.725) (end 126.127 81.899) (width 0.4) (layer F.Cu) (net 14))
 (segment (start 130.105001 93.275001) (end 125.73 88.9) (width 0.4) (layer F.Cu) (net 14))
 (segment (start 130.105001 97.096001) (end 130.105001 93.275001) (width 0.4) (layer F.Cu) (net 14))
 (segment (start 132.087012 99.078012) (end 130.105001 97.096001) (width 0.4) (layer F.Cu) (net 14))
 (segment (start 136.97 113.68) (end 137.769989 112.880011) (width 0.4) (layer F.Cu) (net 14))
 (segment (start 135.57 113.68) (end 136.97 113.68) (width 0.4) (layer F.Cu) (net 14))
 (segment (start 137.769989 112.880011) (end 137.769989 100.192989) (width 0.4) (layer F.Cu) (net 14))
 (segment (start 136.655012 99.078012) (end 132.087012 99.078012) (width 0.4) (layer F.Cu) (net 14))
 (segment (start 137.769989 100.192989) (end 136.655012 99.078012) (width 0.4) (layer F.Cu) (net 14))
 (segment (start 132.08 86.241) (end 132.596 85.725) (width 0.4) (layer F.Cu) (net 13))
 (segment (start 132.08 88.9) (end 132.08 86.241) (width 0.4) (layer F.Cu) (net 13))
 (segment (start 132.596 81.907) (end 133.223 81.28) (width 0.4) (layer F.Cu) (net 13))
 (segment (start 132.596 85.725) (end 132.596 81.907) (width 0.4) (layer F.Cu) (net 13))
 (segment (start 138.369999 113.420001) (end 138.369999 98.506999) (width 0.4) (layer F.Cu) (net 13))
 (segment (start 135.57 116.22) (end 138.369999 113.420001) (width 0.4) (layer F.Cu) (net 13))
 (segment (start 138.369999 98.506999) (end 136.906 97.043) (width 0.4) (layer F.Cu) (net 13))
 (segment (start 136.906 93.726) (end 132.08 88.9) (width 0.4) (layer F.Cu) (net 13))
 (segment (start 136.906 97.043) (end 136.906 93.726) (width 0.4) (layer F.Cu) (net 13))
 (segment (start 138.43 86.36) (end 139.065 85.725) (width 0.4) (layer F.Cu) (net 11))
 (segment (start 138.43 88.9) (end 138.43 86.36) (width 0.4) (layer F.Cu) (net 11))
 (segment (start 139.065 81.915) (end 139.7 81.28) (width 0.4) (layer F.Cu) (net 11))
 (segment (start 139.065 85.725) (end 139.065 81.915) (width 0.4) (layer F.Cu) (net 11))
 (segment (start 135.57 121.3) (end 134.821004 121.3) (width 0.25) (layer F.Cu) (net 11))
 (segment (start 138.43 88.915) (end 138.43 88.9) (width 0.25) (layer F.Cu) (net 11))
 (segment (start 143.570001 94.040001) (end 138.43 88.9) (width 0.4) (layer F.Cu) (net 11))
 (segment (start 143.570001 113.299999) (end 143.570001 94.040001) (width 0.4) (layer F.Cu) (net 11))
 (segment (start 135.57 121.3) (end 143.570001 113.299999) (width 0.4) (layer F.Cu) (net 11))
 (segment (start 142.765001 80.345001) (end 139.7 77.28) (width 0.4) (layer F.Cu) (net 18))
 (segment (start 142.765001 87.739999) (end 142.765001 80.345001) (width 0.4) (layer F.Cu) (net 18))
 (segment (start 141.605 88.9) (end 142.765001 87.739999) (width 0.4) (layer F.Cu) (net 18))
 (segment (start 136.296001 80.353001) (end 133.223 77.28) (width 0.4) (layer F.Cu) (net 19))
 (segment (start 136.296001 87.858999) (end 136.296001 80.353001) (width 0.4) (layer F.Cu) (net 19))
 (segment (start 135.255 88.9) (end 136.296001 87.858999) (width 0.4) (layer F.Cu) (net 19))
 (segment (start 129.827001 80.361001) (end 126.746 77.28) (width 0.4) (layer F.Cu) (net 20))
 (segment (start 129.827001 87.977999) (end 129.827001 80.361001) (width 0.4) (layer F.Cu) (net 20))
 (segment (start 128.905 88.9) (end 129.827001 87.977999) (width 0.4) (layer F.Cu) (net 20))
 (segment (start 123.358001 80.369001) (end 120.269 77.28) (width 0.4) (layer F.Cu) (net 17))
 (segment (start 123.358001 88.096999) (end 123.358001 80.369001) (width 0.4) (layer F.Cu) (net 17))
 (segment (start 122.555 88.9) (end 123.358001 88.096999) (width 0.4) (layer F.Cu) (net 17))
 (segment (start 117.004999 80.492999) (end 113.792 77.28) (width 0.4) (layer F.Cu) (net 21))
 (segment (start 117.004999 88.100001) (end 117.004999 80.492999) (width 0.4) (layer F.Cu) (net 21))
 (segment (start 116.205 88.9) (end 117.004999 88.100001) (width 0.4) (layer F.Cu) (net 21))
 (segment (start 110.654999 88.100001) (end 110.654999 80.619999) (width 0.4) (layer F.Cu) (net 22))
 (segment (start 110.654999 80.619999) (end 107.315 77.28) (width 0.4) (layer F.Cu) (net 22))
 (segment (start 109.855 88.9) (end 110.654999 88.100001) (width 0.4) (layer F.Cu) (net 22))
 (segment (start 136.455001 97.720001) (end 135.255 96.52) (width 0.4) (layer B.Cu) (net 9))
 (segment (start 140.404999 97.720001) (end 136.455001 97.720001) (width 0.4) (layer B.Cu) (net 9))
 (segment (start 141.605 96.52) (end 140.404999 97.720001) (width 0.4) (layer B.Cu) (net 9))
 (segment (start 130.105001 97.720001) (end 128.905 96.52) (width 0.4) (layer B.Cu) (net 9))
 (segment (start 134.054999 97.720001) (end 130.105001 97.720001) (width 0.4) (layer B.Cu) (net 9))
 (segment (start 135.255 96.52) (end 134.054999 97.720001) (width 0.4) (layer B.Cu) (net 9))
 (segment (start 123.755001 97.720001) (end 122.555 96.52) (width 0.4) (layer B.Cu) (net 9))
 (segment (start 127.704999 97.720001) (end 123.755001 97.720001) (width 0.4) (layer B.Cu) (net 9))
 (segment (start 128.905 96.52) (end 127.704999 97.720001) (width 0.4) (layer B.Cu) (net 9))
 (segment (start 117.405001 97.720001) (end 116.205 96.52) (width 0.4) (layer B.Cu) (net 9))
 (segment (start 121.354999 97.720001) (end 117.405001 97.720001) (width 0.4) (layer B.Cu) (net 9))
 (segment (start 122.555 96.52) (end 121.354999 97.720001) (width 0.4) (layer B.Cu) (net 9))
 (segment (start 111.055001 97.720001) (end 109.855 96.52) (width 0.4) (layer B.Cu) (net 9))
 (segment (start 115.004999 97.720001) (end 111.055001 97.720001) (width 0.4) (layer B.Cu) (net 9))
 (segment (start 116.205 96.52) (end 115.004999 97.720001) (width 0.4) (layer B.Cu) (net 9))
 (segment (start 141.605 96.52) (end 143.570001 98.485001) (width 0.4) (layer B.Cu) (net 9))
 (segment (start 143.570001 124.414999) (end 143.570001 98.485001) (width 0.4) (layer B.Cu) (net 9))
 (segment (start 141.605 126.38) (end 143.570001 124.414999) (width 0.4) (layer B.Cu) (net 9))
 (segment (start 135.57 126.38) (end 141.605 126.38) (width 0.4) (layer B.Cu) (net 9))
 (segment (start 111.829999 95.319999) (end 113.03 96.52) (width 0.4) (layer B.Cu) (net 8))
 (segment (start 107.880001 95.319999) (end 111.829999 95.319999) (width 0.4) (layer B.Cu) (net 8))
 (segment (start 106.68 96.52) (end 107.880001 95.319999) (width 0.4) (layer B.Cu) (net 8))
 (segment (start 118.179999 95.319999) (end 119.38 96.52) (width 0.4) (layer B.Cu) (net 8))
 (segment (start 114.230001 95.319999) (end 118.179999 95.319999) (width 0.4) (layer B.Cu) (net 8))
 (segment (start 113.03 96.52) (end 114.230001 95.319999) (width 0.4) (layer B.Cu) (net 8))
 (segment (start 124.529999 95.319999) (end 125.73 96.52) (width 0.4) (layer B.Cu) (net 8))
 (segment (start 120.580001 95.319999) (end 124.529999 95.319999) (width 0.4) (layer B.Cu) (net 8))
 (segment (start 119.38 96.52) (end 120.580001 95.319999) (width 0.4) (layer B.Cu) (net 8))
 (segment (start 130.879999 95.319999) (end 132.08 96.52) (width 0.4) (layer B.Cu) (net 8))
 (segment (start 126.930001 95.319999) (end 130.879999 95.319999) (width 0.4) (layer B.Cu) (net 8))
 (segment (start 125.73 96.52) (end 126.930001 95.319999) (width 0.4) (layer B.Cu) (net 8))
 (segment (start 137.229999 95.319999) (end 138.43 96.52) (width 0.4) (layer B.Cu) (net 8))
 (segment (start 133.280001 95.319999) (end 137.229999 95.319999) (width 0.4) (layer B.Cu) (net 8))
 (segment (start 132.08 96.52) (end 133.280001 95.319999) (width 0.4) (layer B.Cu) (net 8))
 (segment (start 112.71 125.73707) (end 109.915001 122.942071) (width 0.4) (layer B.Cu) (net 8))
 (segment (start 112.71 126.38) (end 112.71 125.73707) (width 0.4) (layer B.Cu) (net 8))
 (segment (start 109.915001 99.755001) (end 106.68 96.52) (width 0.4) (layer B.Cu) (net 8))
 (segment (start 109.915001 122.942071) (end 109.915001 99.755001) (width 0.4) (layer B.Cu) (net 8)))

